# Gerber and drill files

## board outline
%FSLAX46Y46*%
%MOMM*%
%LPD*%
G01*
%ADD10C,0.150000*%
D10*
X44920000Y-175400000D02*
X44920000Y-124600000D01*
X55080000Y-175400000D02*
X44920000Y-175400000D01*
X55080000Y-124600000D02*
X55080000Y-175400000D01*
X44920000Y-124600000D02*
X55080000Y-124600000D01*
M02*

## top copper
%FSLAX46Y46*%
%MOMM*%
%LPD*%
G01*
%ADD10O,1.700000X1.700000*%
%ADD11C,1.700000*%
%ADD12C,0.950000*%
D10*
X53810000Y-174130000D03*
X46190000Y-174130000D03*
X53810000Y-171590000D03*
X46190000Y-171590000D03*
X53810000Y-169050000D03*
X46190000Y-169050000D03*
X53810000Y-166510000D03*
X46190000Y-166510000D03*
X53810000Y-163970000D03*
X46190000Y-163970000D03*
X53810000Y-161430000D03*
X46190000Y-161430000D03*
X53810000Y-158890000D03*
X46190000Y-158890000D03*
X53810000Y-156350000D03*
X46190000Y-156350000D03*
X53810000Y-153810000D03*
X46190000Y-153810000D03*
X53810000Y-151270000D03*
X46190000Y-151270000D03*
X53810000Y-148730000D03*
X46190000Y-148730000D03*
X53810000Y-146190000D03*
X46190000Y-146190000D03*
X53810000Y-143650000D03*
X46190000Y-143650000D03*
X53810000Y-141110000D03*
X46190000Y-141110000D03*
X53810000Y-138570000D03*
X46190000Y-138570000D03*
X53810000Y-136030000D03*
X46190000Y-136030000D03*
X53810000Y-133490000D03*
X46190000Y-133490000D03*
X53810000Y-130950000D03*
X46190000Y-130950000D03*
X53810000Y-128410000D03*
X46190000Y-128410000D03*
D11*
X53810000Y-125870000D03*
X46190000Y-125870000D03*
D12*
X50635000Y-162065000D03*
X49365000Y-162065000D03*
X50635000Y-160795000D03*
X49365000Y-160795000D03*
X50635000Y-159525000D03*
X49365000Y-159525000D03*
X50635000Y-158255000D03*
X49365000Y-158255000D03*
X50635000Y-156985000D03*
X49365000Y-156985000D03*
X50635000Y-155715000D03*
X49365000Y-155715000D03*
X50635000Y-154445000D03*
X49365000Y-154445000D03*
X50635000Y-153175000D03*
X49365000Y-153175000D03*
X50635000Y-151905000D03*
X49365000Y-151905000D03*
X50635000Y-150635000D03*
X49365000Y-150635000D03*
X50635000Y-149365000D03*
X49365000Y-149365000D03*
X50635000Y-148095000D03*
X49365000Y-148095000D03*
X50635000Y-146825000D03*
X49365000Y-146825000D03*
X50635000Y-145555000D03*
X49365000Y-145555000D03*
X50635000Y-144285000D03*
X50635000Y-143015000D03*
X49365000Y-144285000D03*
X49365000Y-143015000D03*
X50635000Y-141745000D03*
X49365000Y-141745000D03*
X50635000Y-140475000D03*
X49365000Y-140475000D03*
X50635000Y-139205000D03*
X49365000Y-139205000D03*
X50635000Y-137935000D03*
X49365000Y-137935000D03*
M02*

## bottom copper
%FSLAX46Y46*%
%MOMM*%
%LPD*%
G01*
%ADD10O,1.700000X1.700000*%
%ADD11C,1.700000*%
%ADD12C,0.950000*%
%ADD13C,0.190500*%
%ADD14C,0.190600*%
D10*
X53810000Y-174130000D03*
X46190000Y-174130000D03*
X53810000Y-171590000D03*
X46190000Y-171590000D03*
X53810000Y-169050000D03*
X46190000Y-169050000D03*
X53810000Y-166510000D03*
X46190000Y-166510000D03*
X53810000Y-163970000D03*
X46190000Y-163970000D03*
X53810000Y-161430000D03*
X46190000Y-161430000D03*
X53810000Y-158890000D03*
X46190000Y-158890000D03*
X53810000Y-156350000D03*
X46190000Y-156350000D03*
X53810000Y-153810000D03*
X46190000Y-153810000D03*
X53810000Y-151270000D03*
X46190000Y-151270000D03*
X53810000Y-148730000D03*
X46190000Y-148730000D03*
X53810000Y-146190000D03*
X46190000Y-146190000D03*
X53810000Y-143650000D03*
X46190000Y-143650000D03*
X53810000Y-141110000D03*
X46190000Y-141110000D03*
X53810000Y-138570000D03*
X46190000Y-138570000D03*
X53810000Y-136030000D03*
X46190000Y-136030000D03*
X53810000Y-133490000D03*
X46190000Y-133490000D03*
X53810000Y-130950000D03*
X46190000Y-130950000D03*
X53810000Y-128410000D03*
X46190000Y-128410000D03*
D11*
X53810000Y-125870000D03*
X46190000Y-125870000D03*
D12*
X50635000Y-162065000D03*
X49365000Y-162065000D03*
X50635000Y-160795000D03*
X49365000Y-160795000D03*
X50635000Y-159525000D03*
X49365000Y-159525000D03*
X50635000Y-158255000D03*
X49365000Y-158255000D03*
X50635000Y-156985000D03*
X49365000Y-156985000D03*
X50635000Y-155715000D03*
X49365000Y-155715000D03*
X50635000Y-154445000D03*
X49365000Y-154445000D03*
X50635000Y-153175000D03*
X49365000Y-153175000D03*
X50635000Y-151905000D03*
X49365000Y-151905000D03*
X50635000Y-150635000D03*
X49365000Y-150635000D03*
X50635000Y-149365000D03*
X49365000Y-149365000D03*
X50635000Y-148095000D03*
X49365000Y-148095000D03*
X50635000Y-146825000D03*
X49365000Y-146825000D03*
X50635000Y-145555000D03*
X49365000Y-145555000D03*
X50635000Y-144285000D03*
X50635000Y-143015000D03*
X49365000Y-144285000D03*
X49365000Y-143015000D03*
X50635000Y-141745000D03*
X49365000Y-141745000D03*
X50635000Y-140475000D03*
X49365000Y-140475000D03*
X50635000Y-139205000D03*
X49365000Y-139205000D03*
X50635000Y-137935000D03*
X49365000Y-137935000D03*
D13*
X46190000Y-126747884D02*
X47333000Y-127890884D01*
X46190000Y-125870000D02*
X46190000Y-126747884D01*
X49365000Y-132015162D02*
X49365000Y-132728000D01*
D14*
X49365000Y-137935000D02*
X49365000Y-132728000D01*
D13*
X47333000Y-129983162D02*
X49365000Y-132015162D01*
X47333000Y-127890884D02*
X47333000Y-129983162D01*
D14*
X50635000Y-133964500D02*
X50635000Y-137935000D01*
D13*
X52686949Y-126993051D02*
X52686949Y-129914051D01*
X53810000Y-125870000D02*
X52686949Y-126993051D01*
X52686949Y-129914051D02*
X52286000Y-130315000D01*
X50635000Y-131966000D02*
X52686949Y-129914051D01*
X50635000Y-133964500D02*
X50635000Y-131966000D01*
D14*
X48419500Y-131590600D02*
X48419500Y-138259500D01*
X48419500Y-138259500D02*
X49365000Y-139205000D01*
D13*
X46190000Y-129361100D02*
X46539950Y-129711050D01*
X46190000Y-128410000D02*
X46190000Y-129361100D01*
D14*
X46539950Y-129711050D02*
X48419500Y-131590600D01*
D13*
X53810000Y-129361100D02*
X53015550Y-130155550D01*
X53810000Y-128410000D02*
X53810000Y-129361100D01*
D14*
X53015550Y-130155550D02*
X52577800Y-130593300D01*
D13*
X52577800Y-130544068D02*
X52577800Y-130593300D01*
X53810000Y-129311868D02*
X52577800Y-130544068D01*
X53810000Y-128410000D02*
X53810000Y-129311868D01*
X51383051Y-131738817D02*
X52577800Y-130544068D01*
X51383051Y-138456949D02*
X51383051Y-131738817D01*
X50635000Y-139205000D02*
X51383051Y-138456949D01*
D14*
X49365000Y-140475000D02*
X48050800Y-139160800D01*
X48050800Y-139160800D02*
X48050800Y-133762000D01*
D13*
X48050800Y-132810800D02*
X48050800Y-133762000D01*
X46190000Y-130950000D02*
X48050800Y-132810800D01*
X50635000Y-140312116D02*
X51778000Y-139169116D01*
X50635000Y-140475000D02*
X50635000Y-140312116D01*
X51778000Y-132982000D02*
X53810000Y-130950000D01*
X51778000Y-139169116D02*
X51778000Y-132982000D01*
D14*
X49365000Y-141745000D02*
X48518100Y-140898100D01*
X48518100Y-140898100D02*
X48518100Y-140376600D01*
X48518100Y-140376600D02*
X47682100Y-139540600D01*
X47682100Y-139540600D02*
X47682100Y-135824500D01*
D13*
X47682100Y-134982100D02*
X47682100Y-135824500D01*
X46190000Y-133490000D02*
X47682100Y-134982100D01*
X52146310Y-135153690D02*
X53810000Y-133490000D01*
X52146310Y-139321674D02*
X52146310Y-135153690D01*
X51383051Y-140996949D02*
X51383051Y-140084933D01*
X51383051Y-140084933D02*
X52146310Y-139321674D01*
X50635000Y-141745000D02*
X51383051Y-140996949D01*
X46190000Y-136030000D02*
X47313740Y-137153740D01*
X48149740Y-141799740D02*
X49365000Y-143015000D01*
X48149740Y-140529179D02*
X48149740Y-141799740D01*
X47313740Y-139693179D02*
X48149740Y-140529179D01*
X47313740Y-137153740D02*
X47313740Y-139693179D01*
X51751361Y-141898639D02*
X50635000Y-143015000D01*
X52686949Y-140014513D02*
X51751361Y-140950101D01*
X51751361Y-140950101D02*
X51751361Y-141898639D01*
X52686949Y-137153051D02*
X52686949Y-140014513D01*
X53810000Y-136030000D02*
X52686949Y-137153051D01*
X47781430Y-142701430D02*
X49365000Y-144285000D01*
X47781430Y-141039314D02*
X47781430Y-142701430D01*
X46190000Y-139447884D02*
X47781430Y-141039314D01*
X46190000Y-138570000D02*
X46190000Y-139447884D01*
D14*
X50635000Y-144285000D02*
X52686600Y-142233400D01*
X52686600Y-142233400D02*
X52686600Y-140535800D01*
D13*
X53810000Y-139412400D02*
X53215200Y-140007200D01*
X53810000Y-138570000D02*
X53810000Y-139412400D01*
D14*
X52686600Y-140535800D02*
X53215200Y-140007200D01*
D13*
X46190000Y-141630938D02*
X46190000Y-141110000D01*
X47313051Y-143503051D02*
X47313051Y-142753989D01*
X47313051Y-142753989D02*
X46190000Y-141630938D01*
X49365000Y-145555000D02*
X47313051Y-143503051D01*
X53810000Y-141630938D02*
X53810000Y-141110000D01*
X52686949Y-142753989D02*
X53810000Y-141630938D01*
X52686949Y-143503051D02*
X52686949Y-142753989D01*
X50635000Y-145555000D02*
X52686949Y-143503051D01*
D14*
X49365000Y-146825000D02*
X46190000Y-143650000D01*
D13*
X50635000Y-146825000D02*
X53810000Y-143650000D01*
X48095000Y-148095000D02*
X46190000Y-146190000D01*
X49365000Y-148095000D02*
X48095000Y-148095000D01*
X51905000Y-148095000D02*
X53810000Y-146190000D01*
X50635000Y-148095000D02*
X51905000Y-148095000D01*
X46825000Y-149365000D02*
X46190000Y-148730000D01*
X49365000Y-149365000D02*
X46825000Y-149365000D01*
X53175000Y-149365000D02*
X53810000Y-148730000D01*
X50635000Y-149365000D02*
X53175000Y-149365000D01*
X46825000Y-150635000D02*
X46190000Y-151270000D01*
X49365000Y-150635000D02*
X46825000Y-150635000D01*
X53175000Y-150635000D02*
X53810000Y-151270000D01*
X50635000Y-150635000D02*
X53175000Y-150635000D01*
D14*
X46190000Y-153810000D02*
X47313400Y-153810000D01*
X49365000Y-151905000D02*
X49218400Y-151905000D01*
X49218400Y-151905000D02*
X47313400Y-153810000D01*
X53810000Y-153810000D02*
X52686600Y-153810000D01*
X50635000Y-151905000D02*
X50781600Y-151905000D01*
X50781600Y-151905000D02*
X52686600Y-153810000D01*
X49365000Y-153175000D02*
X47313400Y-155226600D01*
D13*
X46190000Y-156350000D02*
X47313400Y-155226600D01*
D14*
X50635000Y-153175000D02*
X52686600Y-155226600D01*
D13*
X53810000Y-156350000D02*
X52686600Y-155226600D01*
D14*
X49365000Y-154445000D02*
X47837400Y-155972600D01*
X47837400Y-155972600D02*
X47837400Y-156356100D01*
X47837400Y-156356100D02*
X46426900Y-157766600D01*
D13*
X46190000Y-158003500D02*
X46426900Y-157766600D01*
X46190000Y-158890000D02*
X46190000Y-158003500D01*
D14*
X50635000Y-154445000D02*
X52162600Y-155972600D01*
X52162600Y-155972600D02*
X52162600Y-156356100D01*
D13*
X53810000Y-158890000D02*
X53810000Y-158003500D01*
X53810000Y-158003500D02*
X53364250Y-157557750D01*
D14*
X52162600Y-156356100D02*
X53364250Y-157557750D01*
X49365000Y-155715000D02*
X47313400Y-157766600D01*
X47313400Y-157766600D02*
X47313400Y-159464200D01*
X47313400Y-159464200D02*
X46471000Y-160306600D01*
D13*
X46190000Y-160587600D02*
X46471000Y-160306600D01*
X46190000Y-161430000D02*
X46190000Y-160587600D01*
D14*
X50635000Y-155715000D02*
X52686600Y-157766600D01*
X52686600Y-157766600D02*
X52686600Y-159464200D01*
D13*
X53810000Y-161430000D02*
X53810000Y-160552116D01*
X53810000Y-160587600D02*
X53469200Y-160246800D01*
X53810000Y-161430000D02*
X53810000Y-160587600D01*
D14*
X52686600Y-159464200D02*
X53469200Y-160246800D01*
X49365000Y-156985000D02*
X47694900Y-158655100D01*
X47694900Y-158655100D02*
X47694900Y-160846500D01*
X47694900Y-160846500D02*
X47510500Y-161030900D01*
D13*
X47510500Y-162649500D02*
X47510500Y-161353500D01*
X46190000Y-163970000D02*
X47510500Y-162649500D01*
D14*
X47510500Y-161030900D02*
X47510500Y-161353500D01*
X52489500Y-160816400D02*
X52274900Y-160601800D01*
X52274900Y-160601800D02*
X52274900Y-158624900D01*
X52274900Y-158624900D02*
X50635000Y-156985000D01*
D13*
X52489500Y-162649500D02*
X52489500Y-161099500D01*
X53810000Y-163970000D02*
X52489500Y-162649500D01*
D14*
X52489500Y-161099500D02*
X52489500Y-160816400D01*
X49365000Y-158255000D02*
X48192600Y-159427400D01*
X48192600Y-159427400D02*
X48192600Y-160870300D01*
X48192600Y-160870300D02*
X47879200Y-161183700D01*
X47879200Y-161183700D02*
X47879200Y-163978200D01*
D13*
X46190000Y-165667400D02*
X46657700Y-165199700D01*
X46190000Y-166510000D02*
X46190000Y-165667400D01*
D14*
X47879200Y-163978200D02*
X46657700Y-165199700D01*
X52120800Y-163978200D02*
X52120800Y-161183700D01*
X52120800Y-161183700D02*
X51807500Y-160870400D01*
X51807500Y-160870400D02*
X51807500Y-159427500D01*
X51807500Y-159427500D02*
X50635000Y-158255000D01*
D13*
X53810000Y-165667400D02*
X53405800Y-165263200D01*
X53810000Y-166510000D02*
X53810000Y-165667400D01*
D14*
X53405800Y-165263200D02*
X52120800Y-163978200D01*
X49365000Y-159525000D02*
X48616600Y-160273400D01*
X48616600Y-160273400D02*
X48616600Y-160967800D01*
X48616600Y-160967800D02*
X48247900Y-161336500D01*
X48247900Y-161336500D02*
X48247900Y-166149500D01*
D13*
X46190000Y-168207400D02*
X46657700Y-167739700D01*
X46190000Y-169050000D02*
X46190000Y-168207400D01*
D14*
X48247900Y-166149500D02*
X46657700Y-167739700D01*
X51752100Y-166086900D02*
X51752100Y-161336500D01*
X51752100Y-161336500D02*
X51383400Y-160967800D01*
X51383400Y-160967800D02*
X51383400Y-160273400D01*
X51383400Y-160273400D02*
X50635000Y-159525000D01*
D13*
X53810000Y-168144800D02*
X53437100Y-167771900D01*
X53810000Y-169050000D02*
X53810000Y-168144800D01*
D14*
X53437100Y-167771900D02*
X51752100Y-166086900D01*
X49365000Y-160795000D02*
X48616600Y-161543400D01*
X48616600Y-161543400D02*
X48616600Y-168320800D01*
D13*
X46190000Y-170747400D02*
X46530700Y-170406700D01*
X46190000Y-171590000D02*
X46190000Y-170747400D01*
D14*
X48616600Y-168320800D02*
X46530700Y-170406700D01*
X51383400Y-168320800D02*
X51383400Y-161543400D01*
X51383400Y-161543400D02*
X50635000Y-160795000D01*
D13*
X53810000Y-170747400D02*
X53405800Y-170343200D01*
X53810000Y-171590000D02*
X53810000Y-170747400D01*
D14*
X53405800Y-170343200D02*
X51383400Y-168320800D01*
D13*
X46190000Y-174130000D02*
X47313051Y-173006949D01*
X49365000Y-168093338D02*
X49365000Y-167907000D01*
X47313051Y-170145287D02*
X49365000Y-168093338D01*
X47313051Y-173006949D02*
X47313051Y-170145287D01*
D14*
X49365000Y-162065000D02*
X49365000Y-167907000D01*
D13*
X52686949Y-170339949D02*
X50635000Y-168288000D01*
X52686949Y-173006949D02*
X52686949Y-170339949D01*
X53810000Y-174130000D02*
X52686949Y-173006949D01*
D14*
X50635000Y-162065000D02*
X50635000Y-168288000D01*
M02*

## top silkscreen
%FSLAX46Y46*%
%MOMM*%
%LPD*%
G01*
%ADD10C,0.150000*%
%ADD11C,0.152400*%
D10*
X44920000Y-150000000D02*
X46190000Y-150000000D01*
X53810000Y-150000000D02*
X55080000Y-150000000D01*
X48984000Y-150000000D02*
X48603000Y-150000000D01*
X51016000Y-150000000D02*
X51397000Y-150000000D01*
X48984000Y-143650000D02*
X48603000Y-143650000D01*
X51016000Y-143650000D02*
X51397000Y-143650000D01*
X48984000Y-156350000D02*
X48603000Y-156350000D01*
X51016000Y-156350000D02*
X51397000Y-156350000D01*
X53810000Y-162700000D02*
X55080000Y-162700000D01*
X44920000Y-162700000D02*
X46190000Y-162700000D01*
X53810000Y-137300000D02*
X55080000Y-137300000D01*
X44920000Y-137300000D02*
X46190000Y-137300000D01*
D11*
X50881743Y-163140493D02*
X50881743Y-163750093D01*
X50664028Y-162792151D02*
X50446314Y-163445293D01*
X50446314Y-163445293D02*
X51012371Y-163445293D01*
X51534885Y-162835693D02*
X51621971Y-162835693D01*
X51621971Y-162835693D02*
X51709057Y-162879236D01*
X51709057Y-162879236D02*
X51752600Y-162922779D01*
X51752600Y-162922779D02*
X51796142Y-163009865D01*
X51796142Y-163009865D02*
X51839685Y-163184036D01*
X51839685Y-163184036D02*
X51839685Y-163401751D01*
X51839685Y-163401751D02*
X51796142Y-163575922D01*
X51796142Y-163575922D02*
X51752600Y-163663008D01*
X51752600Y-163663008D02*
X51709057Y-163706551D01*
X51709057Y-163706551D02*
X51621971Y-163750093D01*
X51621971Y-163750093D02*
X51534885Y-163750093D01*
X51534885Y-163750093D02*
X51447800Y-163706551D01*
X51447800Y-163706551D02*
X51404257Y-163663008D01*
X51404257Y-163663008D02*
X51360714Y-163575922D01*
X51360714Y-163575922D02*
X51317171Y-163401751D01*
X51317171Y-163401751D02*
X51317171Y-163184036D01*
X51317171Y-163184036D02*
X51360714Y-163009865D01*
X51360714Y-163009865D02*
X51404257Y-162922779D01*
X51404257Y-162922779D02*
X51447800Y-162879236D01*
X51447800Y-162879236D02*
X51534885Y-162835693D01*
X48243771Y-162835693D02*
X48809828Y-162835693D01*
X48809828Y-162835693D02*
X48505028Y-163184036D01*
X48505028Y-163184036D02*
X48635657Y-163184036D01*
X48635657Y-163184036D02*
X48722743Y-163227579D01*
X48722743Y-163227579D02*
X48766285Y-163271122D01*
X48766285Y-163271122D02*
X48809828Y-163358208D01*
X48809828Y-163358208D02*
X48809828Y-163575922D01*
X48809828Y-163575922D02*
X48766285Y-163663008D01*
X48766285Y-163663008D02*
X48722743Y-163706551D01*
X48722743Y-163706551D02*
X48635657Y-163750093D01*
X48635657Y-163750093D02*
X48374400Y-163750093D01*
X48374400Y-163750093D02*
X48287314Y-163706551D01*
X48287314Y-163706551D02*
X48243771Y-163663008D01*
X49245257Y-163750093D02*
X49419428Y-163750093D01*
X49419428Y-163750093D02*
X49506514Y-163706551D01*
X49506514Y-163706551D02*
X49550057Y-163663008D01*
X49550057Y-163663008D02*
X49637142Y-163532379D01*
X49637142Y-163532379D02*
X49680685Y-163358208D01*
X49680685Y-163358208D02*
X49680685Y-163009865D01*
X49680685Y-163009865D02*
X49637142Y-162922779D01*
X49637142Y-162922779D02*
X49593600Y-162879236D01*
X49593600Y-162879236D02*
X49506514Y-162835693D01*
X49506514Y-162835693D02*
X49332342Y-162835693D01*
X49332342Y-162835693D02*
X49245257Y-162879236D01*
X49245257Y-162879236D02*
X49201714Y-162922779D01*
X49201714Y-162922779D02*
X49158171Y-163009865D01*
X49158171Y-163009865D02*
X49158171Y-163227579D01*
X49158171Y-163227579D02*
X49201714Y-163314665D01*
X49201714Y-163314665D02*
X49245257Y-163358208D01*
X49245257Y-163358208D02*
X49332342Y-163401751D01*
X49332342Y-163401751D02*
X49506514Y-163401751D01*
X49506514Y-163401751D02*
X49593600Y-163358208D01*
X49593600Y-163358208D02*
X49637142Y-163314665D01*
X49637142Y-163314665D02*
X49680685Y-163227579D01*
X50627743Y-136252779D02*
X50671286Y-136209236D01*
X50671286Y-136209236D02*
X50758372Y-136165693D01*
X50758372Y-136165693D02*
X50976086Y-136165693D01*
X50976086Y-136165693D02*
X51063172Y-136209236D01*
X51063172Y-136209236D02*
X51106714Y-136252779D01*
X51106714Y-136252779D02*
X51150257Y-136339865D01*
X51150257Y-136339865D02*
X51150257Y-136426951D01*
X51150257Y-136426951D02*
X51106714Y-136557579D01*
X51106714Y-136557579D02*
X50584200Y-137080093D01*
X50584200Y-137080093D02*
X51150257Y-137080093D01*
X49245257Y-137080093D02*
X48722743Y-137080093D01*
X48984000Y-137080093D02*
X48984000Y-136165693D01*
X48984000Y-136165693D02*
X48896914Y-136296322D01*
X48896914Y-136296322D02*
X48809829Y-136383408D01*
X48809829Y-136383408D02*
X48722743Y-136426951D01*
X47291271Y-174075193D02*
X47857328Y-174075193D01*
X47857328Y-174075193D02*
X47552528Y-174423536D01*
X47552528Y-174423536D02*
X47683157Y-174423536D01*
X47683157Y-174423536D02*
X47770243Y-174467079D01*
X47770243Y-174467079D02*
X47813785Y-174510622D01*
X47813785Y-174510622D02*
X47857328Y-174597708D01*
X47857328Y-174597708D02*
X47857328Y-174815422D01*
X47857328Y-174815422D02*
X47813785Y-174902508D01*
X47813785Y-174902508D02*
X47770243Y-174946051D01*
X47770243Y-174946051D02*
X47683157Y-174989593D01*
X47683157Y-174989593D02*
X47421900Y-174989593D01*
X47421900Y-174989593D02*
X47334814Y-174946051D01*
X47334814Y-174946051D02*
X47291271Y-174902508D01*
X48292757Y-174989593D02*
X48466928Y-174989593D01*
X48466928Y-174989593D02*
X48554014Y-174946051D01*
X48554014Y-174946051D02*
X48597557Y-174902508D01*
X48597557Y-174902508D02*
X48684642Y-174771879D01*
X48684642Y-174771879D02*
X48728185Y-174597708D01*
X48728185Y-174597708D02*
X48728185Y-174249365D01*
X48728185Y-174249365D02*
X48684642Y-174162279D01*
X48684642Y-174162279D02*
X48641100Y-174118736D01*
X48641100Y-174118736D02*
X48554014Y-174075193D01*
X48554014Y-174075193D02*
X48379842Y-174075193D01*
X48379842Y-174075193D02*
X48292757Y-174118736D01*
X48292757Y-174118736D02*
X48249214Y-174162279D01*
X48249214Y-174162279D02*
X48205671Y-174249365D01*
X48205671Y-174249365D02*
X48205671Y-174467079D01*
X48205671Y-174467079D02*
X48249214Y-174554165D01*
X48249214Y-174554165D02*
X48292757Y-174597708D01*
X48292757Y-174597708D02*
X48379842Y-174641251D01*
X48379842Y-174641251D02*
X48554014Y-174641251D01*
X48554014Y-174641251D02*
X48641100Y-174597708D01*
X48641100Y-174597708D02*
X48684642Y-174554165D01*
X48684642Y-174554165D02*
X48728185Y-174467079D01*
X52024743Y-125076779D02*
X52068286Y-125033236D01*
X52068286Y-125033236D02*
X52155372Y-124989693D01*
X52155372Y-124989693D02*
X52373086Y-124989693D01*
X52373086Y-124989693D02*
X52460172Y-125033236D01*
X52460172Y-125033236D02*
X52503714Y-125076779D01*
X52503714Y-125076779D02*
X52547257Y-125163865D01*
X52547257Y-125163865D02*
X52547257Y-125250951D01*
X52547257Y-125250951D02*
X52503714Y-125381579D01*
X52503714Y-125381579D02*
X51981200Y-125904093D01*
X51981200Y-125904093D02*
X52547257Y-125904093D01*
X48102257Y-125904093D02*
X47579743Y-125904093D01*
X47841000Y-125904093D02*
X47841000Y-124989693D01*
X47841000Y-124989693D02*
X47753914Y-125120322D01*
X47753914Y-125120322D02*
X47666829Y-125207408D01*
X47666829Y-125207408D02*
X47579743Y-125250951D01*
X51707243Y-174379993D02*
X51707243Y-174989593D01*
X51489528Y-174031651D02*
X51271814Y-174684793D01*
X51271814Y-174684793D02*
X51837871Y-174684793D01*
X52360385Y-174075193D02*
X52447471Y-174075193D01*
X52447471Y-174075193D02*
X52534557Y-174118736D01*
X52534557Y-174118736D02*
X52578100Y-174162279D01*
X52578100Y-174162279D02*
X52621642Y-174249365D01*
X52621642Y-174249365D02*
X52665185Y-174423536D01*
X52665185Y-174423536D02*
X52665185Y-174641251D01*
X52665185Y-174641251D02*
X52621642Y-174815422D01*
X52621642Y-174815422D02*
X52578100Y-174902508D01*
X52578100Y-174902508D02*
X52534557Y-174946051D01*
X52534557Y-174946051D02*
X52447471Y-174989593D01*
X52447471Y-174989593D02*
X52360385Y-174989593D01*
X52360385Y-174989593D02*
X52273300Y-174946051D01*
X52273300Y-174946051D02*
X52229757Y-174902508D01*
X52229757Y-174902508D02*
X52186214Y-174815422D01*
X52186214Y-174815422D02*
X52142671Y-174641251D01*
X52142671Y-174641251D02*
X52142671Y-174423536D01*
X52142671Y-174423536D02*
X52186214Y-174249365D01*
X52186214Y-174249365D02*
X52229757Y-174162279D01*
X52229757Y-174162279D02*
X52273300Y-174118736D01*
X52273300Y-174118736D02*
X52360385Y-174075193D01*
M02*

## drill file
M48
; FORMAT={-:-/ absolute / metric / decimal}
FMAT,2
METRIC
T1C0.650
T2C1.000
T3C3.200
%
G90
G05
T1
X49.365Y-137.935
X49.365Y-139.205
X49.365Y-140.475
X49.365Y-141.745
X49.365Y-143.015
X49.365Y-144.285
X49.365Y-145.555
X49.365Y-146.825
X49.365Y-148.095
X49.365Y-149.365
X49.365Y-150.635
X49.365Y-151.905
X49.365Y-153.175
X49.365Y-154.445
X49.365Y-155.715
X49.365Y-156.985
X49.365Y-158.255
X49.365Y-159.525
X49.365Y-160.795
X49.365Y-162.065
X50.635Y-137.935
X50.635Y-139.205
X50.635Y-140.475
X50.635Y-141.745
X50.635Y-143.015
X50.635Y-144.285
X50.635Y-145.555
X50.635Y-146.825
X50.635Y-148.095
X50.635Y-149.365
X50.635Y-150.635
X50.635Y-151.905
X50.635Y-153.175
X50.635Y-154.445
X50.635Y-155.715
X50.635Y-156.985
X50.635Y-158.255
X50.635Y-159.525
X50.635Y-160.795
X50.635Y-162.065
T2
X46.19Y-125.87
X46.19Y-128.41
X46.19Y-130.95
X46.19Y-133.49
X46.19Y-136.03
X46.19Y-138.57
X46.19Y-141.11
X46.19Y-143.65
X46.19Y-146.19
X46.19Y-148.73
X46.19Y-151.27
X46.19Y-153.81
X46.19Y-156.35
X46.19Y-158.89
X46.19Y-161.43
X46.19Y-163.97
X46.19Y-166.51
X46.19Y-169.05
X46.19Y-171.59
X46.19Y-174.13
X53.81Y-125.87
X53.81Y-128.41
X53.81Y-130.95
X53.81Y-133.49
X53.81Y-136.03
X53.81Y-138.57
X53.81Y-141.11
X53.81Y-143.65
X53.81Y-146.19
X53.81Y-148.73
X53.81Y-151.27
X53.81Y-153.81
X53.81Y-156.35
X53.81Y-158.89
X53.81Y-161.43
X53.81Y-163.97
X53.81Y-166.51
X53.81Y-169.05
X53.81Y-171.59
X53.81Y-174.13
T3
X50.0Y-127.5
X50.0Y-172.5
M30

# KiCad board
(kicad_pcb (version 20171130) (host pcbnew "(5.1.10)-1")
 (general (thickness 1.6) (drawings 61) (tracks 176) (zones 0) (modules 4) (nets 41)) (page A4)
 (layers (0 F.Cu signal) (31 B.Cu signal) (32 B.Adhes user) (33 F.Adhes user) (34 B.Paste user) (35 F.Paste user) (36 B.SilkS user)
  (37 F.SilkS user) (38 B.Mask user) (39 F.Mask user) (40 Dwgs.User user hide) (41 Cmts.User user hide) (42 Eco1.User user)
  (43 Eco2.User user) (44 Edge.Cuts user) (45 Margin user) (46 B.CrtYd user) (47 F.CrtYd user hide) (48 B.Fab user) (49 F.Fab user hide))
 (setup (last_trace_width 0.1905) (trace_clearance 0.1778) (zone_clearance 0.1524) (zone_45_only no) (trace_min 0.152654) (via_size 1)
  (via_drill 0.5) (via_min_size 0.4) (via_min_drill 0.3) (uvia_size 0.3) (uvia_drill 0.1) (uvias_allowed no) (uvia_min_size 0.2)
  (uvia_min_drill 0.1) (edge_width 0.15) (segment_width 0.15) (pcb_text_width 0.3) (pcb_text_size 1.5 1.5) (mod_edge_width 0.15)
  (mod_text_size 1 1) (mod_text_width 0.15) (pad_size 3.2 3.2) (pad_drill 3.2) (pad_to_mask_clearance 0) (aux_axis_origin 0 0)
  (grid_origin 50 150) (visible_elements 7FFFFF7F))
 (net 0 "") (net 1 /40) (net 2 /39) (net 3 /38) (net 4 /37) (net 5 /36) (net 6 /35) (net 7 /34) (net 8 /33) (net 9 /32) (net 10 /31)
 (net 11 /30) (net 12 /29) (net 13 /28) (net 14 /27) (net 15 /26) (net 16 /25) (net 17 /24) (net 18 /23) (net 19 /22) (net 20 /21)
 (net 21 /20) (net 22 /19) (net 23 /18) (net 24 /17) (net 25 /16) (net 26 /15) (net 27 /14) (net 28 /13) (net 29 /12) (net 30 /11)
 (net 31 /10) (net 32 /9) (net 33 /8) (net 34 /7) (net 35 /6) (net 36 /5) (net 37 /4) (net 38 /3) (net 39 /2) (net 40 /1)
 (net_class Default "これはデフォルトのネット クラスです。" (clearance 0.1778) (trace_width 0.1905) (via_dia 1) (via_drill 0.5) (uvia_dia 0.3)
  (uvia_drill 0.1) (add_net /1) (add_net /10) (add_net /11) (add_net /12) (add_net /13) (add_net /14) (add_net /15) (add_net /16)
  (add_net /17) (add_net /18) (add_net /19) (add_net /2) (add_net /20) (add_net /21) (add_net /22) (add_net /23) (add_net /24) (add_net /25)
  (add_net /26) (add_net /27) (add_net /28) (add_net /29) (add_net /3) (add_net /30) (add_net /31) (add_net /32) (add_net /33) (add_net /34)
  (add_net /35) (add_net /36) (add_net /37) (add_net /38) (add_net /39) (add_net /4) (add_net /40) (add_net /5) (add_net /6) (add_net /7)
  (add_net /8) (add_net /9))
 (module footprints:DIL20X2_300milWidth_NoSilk (layer F.Cu) (at 50 150)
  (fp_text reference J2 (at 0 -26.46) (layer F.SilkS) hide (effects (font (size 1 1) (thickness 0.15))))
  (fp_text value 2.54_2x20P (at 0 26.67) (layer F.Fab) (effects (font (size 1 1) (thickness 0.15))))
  (pad 40 thru_hole oval (at 3.81 24.13) (size 1.7 1.7) (drill 1) (layers *.Cu *.Mask) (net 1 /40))
  (pad 39 thru_hole oval (at -3.81 24.13) (size 1.7 1.7) (drill 1) (layers *.Cu *.Mask) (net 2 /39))
  (pad 38 thru_hole oval (at 3.81 21.59) (size 1.7 1.7) (drill 1) (layers *.Cu *.Mask) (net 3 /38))
  (pad 37 thru_hole oval (at -3.81 21.59) (size 1.7 1.7) (drill 1) (layers *.Cu *.Mask) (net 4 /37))
  (pad 36 thru_hole oval (at 3.81 19.05) (size 1.7 1.7) (drill 1) (layers *.Cu *.Mask) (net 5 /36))
  (pad 35 thru_hole oval (at -3.81 19.05) (size 1.7 1.7) (drill 1) (layers *.Cu *.Mask) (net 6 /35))
  (pad 34 thru_hole oval (at 3.81 16.51) (size 1.7 1.7) (drill 1) (layers *.Cu *.Mask) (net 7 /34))
  (pad 33 thru_hole oval (at -3.81 16.51) (size 1.7 1.7) (drill 1) (layers *.Cu *.Mask) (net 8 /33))
  (pad 32 thru_hole oval (at 3.81 13.97) (size 1.7 1.7) (drill 1) (layers *.Cu *.Mask) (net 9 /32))
  (pad 31 thru_hole oval (at -3.81 13.97) (size 1.7 1.7) (drill 1) (layers *.Cu *.Mask) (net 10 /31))
  (pad 30 thru_hole oval (at 3.81 11.43) (size 1.7 1.7) (drill 1) (layers *.Cu *.Mask) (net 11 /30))
  (pad 29 thru_hole oval (at -3.81 11.43) (size 1.7 1.7) (drill 1) (layers *.Cu *.Mask) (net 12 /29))
  (pad 28 thru_hole oval (at 3.81 8.89) (size 1.7 1.7) (drill 1) (layers *.Cu *.Mask) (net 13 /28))
  (pad 27 thru_hole oval (at -3.81 8.89) (size 1.7 1.7) (drill 1) (layers *.Cu *.Mask) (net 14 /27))
  (pad 26 thru_hole oval (at 3.81 6.35) (size 1.7 1.7) (drill 1) (layers *.Cu *.Mask) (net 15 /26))
  (pad 25 thru_hole oval (at -3.81 6.35) (size 1.7 1.7) (drill 1) (layers *.Cu *.Mask) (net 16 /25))
  (pad 24 thru_hole oval (at 3.81 3.81) (size 1.7 1.7) (drill 1) (layers *.Cu *.Mask) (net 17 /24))
  (pad 23 thru_hole oval (at -3.81 3.81) (size 1.7 1.7) (drill 1) (layers *.Cu *.Mask) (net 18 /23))
  (pad 22 thru_hole oval (at 3.81 1.27) (size 1.7 1.7) (drill 1) (layers *.Cu *.Mask) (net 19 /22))
  (pad 21 thru_hole oval (at -3.81 1.27) (size 1.7 1.7) (drill 1) (layers *.Cu *.Mask) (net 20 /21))
  (pad 20 thru_hole oval (at 3.81 -1.27) (size 1.7 1.7) (drill 1) (layers *.Cu *.Mask) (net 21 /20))
  (pad 19 thru_hole oval (at -3.81 -1.27) (size 1.7 1.7) (drill 1) (layers *.Cu *.Mask) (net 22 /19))
  (pad 18 thru_hole oval (at 3.81 -3.81) (size 1.7 1.7) (drill 1) (layers *.Cu *.Mask) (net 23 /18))
  (pad 17 thru_hole oval (at -3.81 -3.81) (size 1.7 1.7) (drill 1) (layers *.Cu *.Mask) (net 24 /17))
  (pad 16 thru_hole oval (at 3.81 -6.35) (size 1.7 1.7) (drill 1) (layers *.Cu *.Mask) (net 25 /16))
  (pad 15 thru_hole oval (at -3.81 -6.35) (size 1.7 1.7) (drill 1) (layers *.Cu *.Mask) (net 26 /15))
  (pad 14 thru_hole oval (at 3.81 -8.89) (size 1.7 1.7) (drill 1) (layers *.Cu *.Mask) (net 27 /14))
  (pad 13 thru_hole oval (at -3.81 -8.89) (size 1.7 1.7) (drill 1) (layers *.Cu *.Mask) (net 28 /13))
  (pad 12 thru_hole oval (at 3.81 -11.43) (size 1.7 1.7) (drill 1) (layers *.Cu *.Mask) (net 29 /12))
  (pad 11 thru_hole oval (at -3.81 -11.43) (size 1.7 1.7) (drill 1) (layers *.Cu *.Mask) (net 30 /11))
  (pad 10 thru_hole oval (at 3.81 -13.97) (size 1.7 1.7) (drill 1) (layers *.Cu *.Mask) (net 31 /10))
  (pad 9 thru_hole oval (at -3.81 -13.97) (size 1.7 1.7) (drill 1) (layers *.Cu *.Mask) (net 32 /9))
  (pad 8 thru_hole oval (at 3.81 -16.51) (size 1.7 1.7) (drill 1) (layers *.Cu *.Mask) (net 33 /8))
  (pad 7 thru_hole oval (at -3.81 -16.51) (size 1.7 1.7) (drill 1) (layers *.Cu *.Mask) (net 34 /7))
  (pad 6 thru_hole oval (at 3.81 -19.05) (size 1.7 1.7) (drill 1) (layers *.Cu *.Mask) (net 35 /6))
  (pad 5 thru_hole oval (at -3.81 -19.05) (size 1.7 1.7) (drill 1) (layers *.Cu *.Mask) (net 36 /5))
  (pad 4 thru_hole oval (at 3.81 -21.59) (size 1.7 1.7) (drill 1) (layers *.Cu *.Mask) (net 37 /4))
  (pad 3 thru_hole oval (at -3.81 -21.59) (size 1.7 1.7) (drill 1) (layers *.Cu *.Mask) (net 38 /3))
  (pad 2 thru_hole circle (at 3.81 -24.13) (size 1.7 1.7) (drill 1) (layers *.Cu *.Mask) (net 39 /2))
  (pad 1 thru_hole circle (at -3.81 -24.13) (size 1.7 1.7) (drill 1) (layers *.Cu *.Mask) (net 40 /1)))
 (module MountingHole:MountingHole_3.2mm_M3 (layer F.Cu) (at 50 127)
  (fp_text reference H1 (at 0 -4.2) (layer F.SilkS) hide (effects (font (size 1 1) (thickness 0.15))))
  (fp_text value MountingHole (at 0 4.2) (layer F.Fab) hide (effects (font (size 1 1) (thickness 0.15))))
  (pad "" np_thru_hole circle (at 0 0.5) (size 3.2 3.2) (drill 3.2) (layers *.Cu *.Mask)))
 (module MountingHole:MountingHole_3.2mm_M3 (layer F.Cu) (at 50 173)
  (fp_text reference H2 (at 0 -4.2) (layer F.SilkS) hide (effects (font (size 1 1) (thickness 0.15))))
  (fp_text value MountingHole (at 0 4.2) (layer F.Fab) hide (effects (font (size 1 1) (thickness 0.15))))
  (pad "" np_thru_hole circle (at 0 -0.5) (size 3.2 3.2) (drill 3.2) (layers *.Cu *.Mask)))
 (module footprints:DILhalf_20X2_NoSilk (layer F.Cu) (at 50 150)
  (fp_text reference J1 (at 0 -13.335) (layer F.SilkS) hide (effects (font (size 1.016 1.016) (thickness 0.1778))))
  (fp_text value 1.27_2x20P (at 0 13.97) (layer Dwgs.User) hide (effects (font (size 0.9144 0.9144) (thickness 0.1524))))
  (pad 40 thru_hole circle (at 0.635 12.065) (size 0.95 0.95) (drill 0.65) (layers *.Cu *.Mask) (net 1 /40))
  (pad 39 thru_hole circle (at -0.635 12.065) (size 0.95 0.95) (drill 0.65) (layers *.Cu *.Mask) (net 2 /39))
  (pad 38 thru_hole circle (at 0.635 10.795) (size 0.95 0.95) (drill 0.65) (layers *.Cu *.Mask) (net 3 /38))
  (pad 37 thru_hole circle (at -0.635 10.795) (size 0.95 0.95) (drill 0.65) (layers *.Cu *.Mask) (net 4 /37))
  (pad 36 thru_hole circle (at 0.635 9.525) (size 0.95 0.95) (drill 0.65) (layers *.Cu *.Mask) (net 5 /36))
  (pad 35 thru_hole circle (at -0.635 9.525) (size 0.95 0.95) (drill 0.65) (layers *.Cu *.Mask) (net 6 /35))
  (pad 34 thru_hole circle (at 0.635 8.255) (size 0.95 0.95) (drill 0.65) (layers *.Cu *.Mask) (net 7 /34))
  (pad 33 thru_hole circle (at -0.635 8.255) (size 0.95 0.95) (drill 0.65) (layers *.Cu *.Mask) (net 8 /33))
  (pad 32 thru_hole circle (at 0.635 6.985) (size 0.95 0.95) (drill 0.65) (layers *.Cu *.Mask) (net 9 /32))
  (pad 31 thru_hole circle (at -0.635 6.985) (size 0.95 0.95) (drill 0.65) (layers *.Cu *.Mask) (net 10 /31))
  (pad 30 thru_hole circle (at 0.635 5.715) (size 0.95 0.95) (drill 0.65) (layers *.Cu *.Mask) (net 11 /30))
  (pad 29 thru_hole circle (at -0.635 5.715) (size 0.95 0.95) (drill 0.65) (layers *.Cu *.Mask) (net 12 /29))
  (pad 28 thru_hole circle (at 0.635 4.445) (size 0.95 0.95) (drill 0.65) (layers *.Cu *.Mask) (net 13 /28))
  (pad 27 thru_hole circle (at -0.635 4.445) (size 0.95 0.95) (drill 0.65) (layers *.Cu *.Mask) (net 14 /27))
  (pad 26 thru_hole circle (at 0.635 3.175) (size 0.95 0.95) (drill 0.65) (layers *.Cu *.Mask) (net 15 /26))
  (pad 25 thru_hole circle (at -0.635 3.175) (size 0.95 0.95) (drill 0.65) (layers *.Cu *.Mask) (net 16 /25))
  (pad 24 thru_hole circle (at 0.635 1.905) (size 0.95 0.95) (drill 0.65) (layers *.Cu *.Mask) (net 17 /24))
  (pad 23 thru_hole circle (at -0.635 1.905) (size 0.95 0.95) (drill 0.65) (layers *.Cu *.Mask) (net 18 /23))
  (pad 22 thru_hole circle (at 0.635 0.635) (size 0.95 0.95) (drill 0.65) (layers *.Cu *.Mask) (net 19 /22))
  (pad 21 thru_hole circle (at -0.635 0.635) (size 0.95 0.95) (drill 0.65) (layers *.Cu *.Mask) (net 20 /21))
  (pad 20 thru_hole circle (at 0.635 -0.635) (size 0.95 0.95) (drill 0.65) (layers *.Cu *.Mask) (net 21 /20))
  (pad 19 thru_hole circle (at -0.635 -0.635) (size 0.95 0.95) (drill 0.65) (layers *.Cu *.Mask) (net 22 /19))
  (pad 18 thru_hole circle (at 0.635 -1.905) (size 0.95 0.95) (drill 0.65) (layers *.Cu *.Mask) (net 23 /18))
  (pad 17 thru_hole circle (at -0.635 -1.905) (size 0.95 0.95) (drill 0.65) (layers *.Cu *.Mask) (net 24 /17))
  (pad 16 thru_hole circle (at 0.635 -3.175) (size 0.95 0.95) (drill 0.65) (layers *.Cu *.Mask) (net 25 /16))
  (pad 15 thru_hole circle (at -0.635 -3.175) (size 0.95 0.95) (drill 0.65) (layers *.Cu *.Mask) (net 26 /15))
  (pad 14 thru_hole circle (at 0.635 -4.445) (size 0.95 0.95) (drill 0.65) (layers *.Cu *.Mask) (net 27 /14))
  (pad 13 thru_hole circle (at -0.635 -4.445) (size 0.95 0.95) (drill 0.65) (layers *.Cu *.Mask) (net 28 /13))
  (pad 12 thru_hole circle (at 0.635 -5.715) (size 0.95 0.95) (drill 0.65) (layers *.Cu *.Mask) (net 29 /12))
  (pad 10 thru_hole circle (at 0.635 -6.985) (size 0.95 0.95) (drill 0.65) (layers *.Cu *.Mask) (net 31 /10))
  (pad 11 thru_hole circle (at -0.635 -5.715) (size 0.95 0.95) (drill 0.65) (layers *.Cu *.Mask) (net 30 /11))
  (pad 9 thru_hole circle (at -0.635 -6.985) (size 0.95 0.95) (drill 0.65) (layers *.Cu *.Mask) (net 32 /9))
  (pad 8 thru_hole circle (at 0.635 -8.255) (size 0.95 0.95) (drill 0.65) (layers *.Cu *.Mask) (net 33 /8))
  (pad 7 thru_hole circle (at -0.635 -8.255) (size 0.95 0.95) (drill 0.65) (layers *.Cu *.Mask) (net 34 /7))
  (pad 6 thru_hole circle (at 0.635 -9.525) (size 0.95 0.95) (drill 0.65) (layers *.Cu *.Mask) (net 35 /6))
  (pad 5 thru_hole circle (at -0.635 -9.525) (size 0.95 0.95) (drill 0.65) (layers *.Cu *.Mask) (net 36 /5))
  (pad 4 thru_hole circle (at 0.635 -10.795) (size 0.95 0.95) (drill 0.65) (layers *.Cu *.Mask) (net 37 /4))
  (pad 3 thru_hole circle (at -0.635 -10.795) (size 0.95 0.95) (drill 0.65) (layers *.Cu *.Mask) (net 38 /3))
  (pad 2 thru_hole circle (at 0.635 -12.065) (size 0.95 0.95) (drill 0.65) (layers *.Cu *.Mask) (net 39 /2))
  (pad 1 thru_hole circle (at -0.635 -12.065) (size 0.95 0.95) (drill 0.65) (layers *.Cu *.Mask) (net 40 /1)))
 (gr_line (start 44.92 150) (end 46.19 150) (layer F.SilkS) (width 0.15))
 (gr_line (start 53.81 150) (end 55.08 150) (layer F.SilkS) (width 0.15))
 (gr_line (start 48.984 150) (end 48.603 150) (layer F.SilkS) (width 0.15))
 (gr_line (start 51.016 150) (end 51.397 150) (layer F.SilkS) (width 0.15))
 (gr_line (start 48.984 143.65) (end 48.603 143.65) (layer F.SilkS) (width 0.15))
 (gr_line (start 51.016 143.65) (end 51.397 143.65) (layer F.SilkS) (width 0.15))
 (gr_line (start 48.984 156.35) (end 48.603 156.35) (layer F.SilkS) (width 0.15))
 (gr_line (start 51.016 156.35) (end 51.397 156.35) (layer F.SilkS) (width 0.15))
 (gr_line (start 53.81 162.7) (end 55.08 162.7) (layer F.SilkS) (width 0.15))
 (gr_line (start 44.92 162.7) (end 46.19 162.7) (layer F.SilkS) (width 0.15))
 (gr_line (start 53.81 137.3) (end 55.08 137.3) (layer F.SilkS) (width 0.15))
 (gr_line (start 44.92 137.3) (end 46.19 137.3) (layer F.SilkS) (width 0.15))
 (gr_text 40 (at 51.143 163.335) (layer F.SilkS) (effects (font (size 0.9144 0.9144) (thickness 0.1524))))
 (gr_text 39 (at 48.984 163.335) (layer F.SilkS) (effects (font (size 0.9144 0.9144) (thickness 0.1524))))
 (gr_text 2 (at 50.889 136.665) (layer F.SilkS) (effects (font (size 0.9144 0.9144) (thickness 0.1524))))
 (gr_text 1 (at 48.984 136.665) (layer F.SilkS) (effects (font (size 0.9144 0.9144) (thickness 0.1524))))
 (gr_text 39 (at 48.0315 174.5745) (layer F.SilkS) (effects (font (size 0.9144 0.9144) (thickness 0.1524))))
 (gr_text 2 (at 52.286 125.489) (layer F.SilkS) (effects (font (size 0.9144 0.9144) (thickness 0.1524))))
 (gr_line (start 44.92 175.4) (end 44.92 124.6) (layer Edge.Cuts) (width 0.15))
 (gr_line (start 55.08 175.4) (end 44.92 175.4) (layer Edge.Cuts) (width 0.15))
 (gr_line (start 55.08 124.6) (end 55.08 175.4) (layer Edge.Cuts) (width 0.15))
 (gr_line (start 44.92 124.6) (end 55.08 124.6) (layer Edge.Cuts) (width 0.15))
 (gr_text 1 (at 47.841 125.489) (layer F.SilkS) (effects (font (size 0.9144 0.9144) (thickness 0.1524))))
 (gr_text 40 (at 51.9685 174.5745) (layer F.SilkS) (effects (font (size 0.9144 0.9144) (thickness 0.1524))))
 (segment (start 46.19 126.747884) (end 47.333 127.890884) (width 0.1905) (layer B.Cu) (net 40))
 (segment (start 46.19 125.87) (end 46.19 126.747884) (width 0.1905) (layer B.Cu) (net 40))
 (segment (start 49.365 132.015162) (end 49.365 132.728) (width 0.1905) (layer B.Cu) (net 40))
 (segment (start 49.365 137.935) (end 49.365 132.728) (width 0.1906) (layer B.Cu) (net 40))
 (segment (start 47.333 129.983162) (end 49.365 132.015162) (width 0.1905) (layer B.Cu) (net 40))
 (segment (start 47.333 127.890884) (end 47.333 129.983162) (width 0.1905) (layer B.Cu) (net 40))
 (segment (start 50.635 133.9645) (end 50.635 137.935) (width 0.1906) (layer B.Cu) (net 39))
 (segment (start 52.686949 126.993051) (end 52.686949 129.914051) (width 0.1905) (layer B.Cu) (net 39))
 (segment (start 53.81 125.87) (end 52.686949 126.993051) (width 0.1905) (layer B.Cu) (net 39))
 (segment (start 52.686949 129.914051) (end 52.286 130.315) (width 0.1905) (layer B.Cu) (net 39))
 (segment (start 50.635 131.966) (end 52.686949 129.914051) (width 0.1905) (layer B.Cu) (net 39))
 (segment (start 50.635 133.9645) (end 50.635 131.966) (width 0.1905) (layer B.Cu) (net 39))
 (segment (start 48.4195 131.5906) (end 48.4195 138.2595) (width 0.1906) (layer B.Cu) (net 38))
 (segment (start 48.4195 138.2595) (end 49.365 139.205) (width 0.1906) (layer B.Cu) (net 38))
 (segment (start 46.19 129.3611) (end 46.53995 129.71105) (width 0.1905) (layer B.Cu) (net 38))
 (segment (start 46.19 128.41) (end 46.19 129.3611) (width 0.1905) (layer B.Cu) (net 38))
 (segment (start 46.53995 129.71105) (end 48.4195 131.5906) (width 0.1906) (layer B.Cu) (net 38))
 (segment (start 53.81 129.3611) (end 53.01555 130.15555) (width 0.1905) (layer B.Cu) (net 37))
 (segment (start 53.81 128.41) (end 53.81 129.3611) (width 0.1905) (layer B.Cu) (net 37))
 (segment (start 53.01555 130.15555) (end 52.5778 130.5933) (width 0.1906) (layer B.Cu) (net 37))
 (segment (start 52.5778 130.544068) (end 52.5778 130.5933) (width 0.1905) (layer B.Cu) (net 37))
 (segment (start 53.81 129.311868) (end 52.5778 130.544068) (width 0.1905) (layer B.Cu) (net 37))
 (segment (start 53.81 128.41) (end 53.81 129.311868) (width 0.1905) (layer B.Cu) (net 37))
 (segment (start 51.383051 131.738817) (end 52.5778 130.544068) (width 0.1905) (layer B.Cu) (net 37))
 (segment (start 51.383051 138.456949) (end 51.383051 131.738817) (width 0.1905) (layer B.Cu) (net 37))
 (segment (start 50.635 139.205) (end 51.383051 138.456949) (width 0.1905) (layer B.Cu) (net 37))
 (segment (start 49.365 140.475) (end 48.0508 139.1608) (width 0.1906) (layer B.Cu) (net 36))
 (segment (start 48.0508 139.1608) (end 48.0508 133.762) (width 0.1906) (layer B.Cu) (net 36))
 (segment (start 48.0508 132.8108) (end 48.0508 133.762) (width 0.1905) (layer B.Cu) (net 36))
 (segment (start 46.19 130.95) (end 48.0508 132.8108) (width 0.1905) (layer B.Cu) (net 36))
 (segment (start 50.635 140.312116) (end 51.778 139.169116) (width 0.1905) (layer B.Cu) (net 35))
 (segment (start 50.635 140.475) (end 50.635 140.312116) (width 0.1905) (layer B.Cu) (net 35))
 (segment (start 51.778 132.982) (end 53.81 130.95) (width 0.1905) (layer B.Cu) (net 35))
 (segment (start 51.778 139.169116) (end 51.778 132.982) (width 0.1905) (layer B.Cu) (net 35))
 (segment (start 49.365 141.745) (end 48.5181 140.8981) (width 0.1906) (layer B.Cu) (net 34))
 (segment (start 48.5181 140.8981) (end 48.5181 140.3766) (width 0.1906) (layer B.Cu) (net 34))
 (segment (start 48.5181 140.3766) (end 47.6821 139.5406) (width 0.1906) (layer B.Cu) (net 34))
 (segment (start 47.6821 139.5406) (end 47.6821 135.8245) (width 0.1906) (layer B.Cu) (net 34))
 (segment (start 47.6821 134.9821) (end 47.6821 135.8245) (width 0.1905) (layer B.Cu) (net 34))
 (segment (start 46.19 133.49) (end 47.6821 134.9821) (width 0.1905) (layer B.Cu) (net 34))
 (segment (start 52.14631 135.15369) (end 53.81 133.49) (width 0.1905) (layer B.Cu) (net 33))
 (segment (start 52.14631 139.321674) (end 52.14631 135.15369) (width 0.1905) (layer B.Cu) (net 33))
 (segment (start 51.383051 140.996949) (end 51.383051 140.084933) (width 0.1905) (layer B.Cu) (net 33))
 (segment (start 51.383051 140.084933) (end 52.14631 139.321674) (width 0.1905) (layer B.Cu) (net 33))
 (segment (start 50.635 141.745) (end 51.383051 140.996949) (width 0.1905) (layer B.Cu) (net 33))
 (segment (start 46.19 136.03) (end 47.31374 137.15374) (width 0.1905) (layer B.Cu) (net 32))
 (segment (start 48.14974 141.79974) (end 49.365 143.015) (width 0.1905) (layer B.Cu) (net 32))
 (segment (start 48.14974 140.529179) (end 48.14974 141.79974) (width 0.1905) (layer B.Cu) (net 32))
 (segment (start 47.31374 139.693179) (end 48.14974 140.529179) (width 0.1905) (layer B.Cu) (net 32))
 (segment (start 47.31374 137.15374) (end 47.31374 139.693179) (width 0.1905) (layer B.Cu) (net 32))
 (segment (start 51.751361 141.898639) (end 50.635 143.015) (width 0.1905) (layer B.Cu) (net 31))
 (segment (start 52.686949 140.014513) (end 51.751361 140.950101) (width 0.1905) (layer B.Cu) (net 31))
 (segment (start 51.751361 140.950101) (end 51.751361 141.898639) (width 0.1905) (layer B.Cu) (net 31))
 (segment (start 52.686949 137.153051) (end 52.686949 140.014513) (width 0.1905) (layer B.Cu) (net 31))
 (segment (start 53.81 136.03) (end 52.686949 137.153051) (width 0.1905) (layer B.Cu) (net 31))
 (segment (start 47.78143 142.70143) (end 49.365 144.285) (width 0.1905) (layer B.Cu) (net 30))
 (segment (start 47.78143 141.039314) (end 47.78143 142.70143) (width 0.1905) (layer B.Cu) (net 30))
 (segment (start 46.19 139.447884) (end 47.78143 141.039314) (width 0.1905) (layer B.Cu) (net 30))
 (segment (start 46.19 138.57) (end 46.19 139.447884) (width 0.1905) (layer B.Cu) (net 30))
 (segment (start 50.635 144.285) (end 52.6866 142.2334) (width 0.1906) (layer B.Cu) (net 29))
 (segment (start 52.6866 142.2334) (end 52.6866 140.5358) (width 0.1906) (layer B.Cu) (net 29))
 (segment (start 53.81 139.4124) (end 53.2152 140.0072) (width 0.1905) (layer B.Cu) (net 29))
 (segment (start 53.81 138.57) (end 53.81 139.4124) (width 0.1905) (layer B.Cu) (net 29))
 (segment (start 52.6866 140.5358) (end 53.2152 140.0072) (width 0.1906) (layer B.Cu) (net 29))
 (segment (start 46.19 141.630938) (end 46.19 141.11) (width 0.1905) (layer B.Cu) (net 28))
 (segment (start 47.313051 143.503051) (end 47.313051 142.753989) (width 0.1905) (layer B.Cu) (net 28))
 (segment (start 47.313051 142.753989) (end 46.19 141.630938) (width 0.1905) (layer B.Cu) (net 28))
 (segment (start 49.365 145.555) (end 47.313051 143.503051) (width 0.1905) (layer B.Cu) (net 28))
 (segment (start 53.81 141.630938) (end 53.81 141.11) (width 0.1905) (layer B.Cu) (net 27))
 (segment (start 52.686949 142.753989) (end 53.81 141.630938) (width 0.1905) (layer B.Cu) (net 27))
 (segment (start 52.686949 143.503051) (end 52.686949 142.753989) (width 0.1905) (layer B.Cu) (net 27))
 (segment (start 50.635 145.555) (end 52.686949 143.503051) (width 0.1905) (layer B.Cu) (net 27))
 (segment (start 49.365 146.825) (end 46.19 143.65) (width 0.1906) (layer B.Cu) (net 26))
 (segment (start 50.635 146.825) (end 53.81 143.65) (width 0.1905) (layer B.Cu) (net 25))
 (segment (start 48.095 148.095) (end 46.19 146.19) (width 0.1905) (layer B.Cu) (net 24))
 (segment (start 49.365 148.095) (end 48.095 148.095) (width 0.1905) (layer B.Cu) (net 24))
 (segment (start 51.905 148.095) (end 53.81 146.19) (width 0.1905) (layer B.Cu) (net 23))
 (segment (start 50.635 148.095) (end 51.905 148.095) (width 0.1905) (layer B.Cu) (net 23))
 (segment (start 46.825 149.365) (end 46.19 148.73) (width 0.1905) (layer B.Cu) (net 22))
 (segment (start 49.365 149.365) (end 46.825 149.365) (width 0.1905) (layer B.Cu) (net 22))
 (segment (start 53.175 149.365) (end 53.81 148.73) (width 0.1905) (layer B.Cu) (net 21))
 (segment (start 50.635 149.365) (end 53.175 149.365) (width 0.1905) (layer B.Cu) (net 21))
 (segment (start 46.825 150.635) (end 46.19 151.27) (width 0.1905) (layer B.Cu) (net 20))
 (segment (start 49.365 150.635) (end 46.825 150.635) (width 0.1905) (layer B.Cu) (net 20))
 (segment (start 53.175 150.635) (end 53.81 151.27) (width 0.1905) (layer B.Cu) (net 19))
 (segment (start 50.635 150.635) (end 53.175 150.635) (width 0.1905) (layer B.Cu) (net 19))
 (segment (start 46.19 153.81) (end 47.3134 153.81) (width 0.1906) (layer B.Cu) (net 18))
 (segment (start 49.365 151.905) (end 49.2184 151.905) (width 0.1906) (layer B.Cu) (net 18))
 (segment (start 49.2184 151.905) (end 47.3134 153.81) (width 0.1906) (layer B.Cu) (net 18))
 (segment (start 53.81 153.81) (end 52.6866 153.81) (width 0.1906) (layer B.Cu) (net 17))
 (segment (start 50.635 151.905) (end 50.7816 151.905) (width 0.1906) (layer B.Cu) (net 17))
 (segment (start 50.7816 151.905) (end 52.6866 153.81) (width 0.1906) (layer B.Cu) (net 17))
 (segment (start 49.365 153.175) (end 47.3134 155.2266) (width 0.1906) (layer B.Cu) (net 16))
 (segment (start 46.19 156.35) (end 47.3134 155.2266) (width 0.1905) (layer B.Cu) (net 16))
 (segment (start 50.635 153.175) (end 52.6866 155.2266) (width 0.1906) (layer B.Cu) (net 15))
 (segment (start 53.81 156.35) (end 52.6866 155.2266) (width 0.1905) (layer B.Cu) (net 15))
 (segment (start 49.365 154.445) (end 47.8374 155.9726) (width 0.1906) (layer B.Cu) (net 14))
 (segment (start 47.8374 155.9726) (end 47.8374 156.3561) (width 0.1906) (layer B.Cu) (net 14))
 (segment (start 47.8374 156.3561) (end 46.4269 157.7666) (width 0.1906) (layer B.Cu) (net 14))
 (segment (start 46.19 158.0035) (end 46.4269 157.7666) (width 0.1905) (layer B.Cu) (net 14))
 (segment (start 46.19 158.89) (end 46.19 158.0035) (width 0.1905) (layer B.Cu) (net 14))
 (segment (start 50.635 154.445) (end 52.1626 155.9726) (width 0.1906) (layer B.Cu) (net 13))
 (segment (start 52.1626 155.9726) (end 52.1626 156.3561) (width 0.1906) (layer B.Cu) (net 13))
 (segment (start 53.81 158.89) (end 53.81 158.0035) (width 0.1905) (layer B.Cu) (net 13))
 (segment (start 53.81 158.0035) (end 53.36425 157.55775) (width 0.1905) (layer B.Cu) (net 13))
 (segment (start 52.1626 156.3561) (end 53.36425 157.55775) (width 0.1906) (layer B.Cu) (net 13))
 (segment (start 49.365 155.715) (end 47.3134 157.7666) (width 0.1906) (layer B.Cu) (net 12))
 (segment (start 47.3134 157.7666) (end 47.3134 159.4642) (width 0.1906) (layer B.Cu) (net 12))
 (segment (start 47.3134 159.4642) (end 46.471 160.3066) (width 0.1906) (layer B.Cu) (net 12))
 (segment (start 46.19 160.5876) (end 46.471 160.3066) (width 0.1905) (layer B.Cu) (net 12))
 (segment (start 46.19 161.43) (end 46.19 160.5876) (width 0.1905) (layer B.Cu) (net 12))
 (segment (start 50.635 155.715) (end 52.6866 157.7666) (width 0.1906) (layer B.Cu) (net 11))
 (segment (start 52.6866 157.7666) (end 52.6866 159.4642) (width 0.1906) (layer B.Cu) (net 11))
 (segment (start 53.81 161.43) (end 53.81 160.552116) (width 0.1905) (layer B.Cu) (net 11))
 (segment (start 53.81 160.5876) (end 53.4692 160.2468) (width 0.1905) (layer B.Cu) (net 11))
 (segment (start 53.81 161.43) (end 53.81 160.5876) (width 0.1905) (layer B.Cu) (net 11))
 (segment (start 52.6866 159.4642) (end 53.4692 160.2468) (width 0.1906) (layer B.Cu) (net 11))
 (segment (start 49.365 156.985) (end 47.6949 158.6551) (width 0.1906) (layer B.Cu) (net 10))
 (segment (start 47.6949 158.6551) (end 47.6949 160.8465) (width 0.1906) (layer B.Cu) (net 10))
 (segment (start 47.6949 160.8465) (end 47.5105 161.0309) (width 0.1906) (layer B.Cu) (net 10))
 (segment (start 47.5105 162.6495) (end 47.5105 161.3535) (width 0.1905) (layer B.Cu) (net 10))
 (segment (start 46.19 163.97) (end 47.5105 162.6495) (width 0.1905) (layer B.Cu) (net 10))
 (segment (start 47.5105 161.0309) (end 47.5105 161.3535) (width 0.1906) (layer B.Cu) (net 10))
 (segment (start 52.4895 160.8164) (end 52.2749 160.6018) (width 0.1906) (layer B.Cu) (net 9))
 (segment (start 52.2749 160.6018) (end 52.2749 158.6249) (width 0.1906) (layer B.Cu) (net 9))
 (segment (start 52.2749 158.6249) (end 50.635 156.985) (width 0.1906) (layer B.Cu) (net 9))
 (segment (start 52.4895 162.6495) (end 52.4895 161.0995) (width 0.1905) (layer B.Cu) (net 9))
 (segment (start 53.81 163.97) (end 52.4895 162.6495) (width 0.1905) (layer B.Cu) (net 9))
 (segment (start 52.4895 161.0995) (end 52.4895 160.8164) (width 0.1906) (layer B.Cu) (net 9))
 (segment (start 49.365 158.255) (end 48.1926 159.4274) (width 0.1906) (layer B.Cu) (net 8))
 (segment (start 48.1926 159.4274) (end 48.1926 160.8703) (width 0.1906) (layer B.Cu) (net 8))
 (segment (start 48.1926 160.8703) (end 47.8792 161.1837) (width 0.1906) (layer B.Cu) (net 8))
 (segment (start 47.8792 161.1837) (end 47.8792 163.9782) (width 0.1906) (layer B.Cu) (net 8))
 (segment (start 46.19 165.6674) (end 46.6577 165.1997) (width 0.1905) (layer B.Cu) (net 8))
 (segment (start 46.19 166.51) (end 46.19 165.6674) (width 0.1905) (layer B.Cu) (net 8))
 (segment (start 47.8792 163.9782) (end 46.6577 165.1997) (width 0.1906) (layer B.Cu) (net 8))
 (segment (start 52.1208 163.9782) (end 52.1208 161.1837) (width 0.1906) (layer B.Cu) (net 7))
 (segment (start 52.1208 161.1837) (end 51.8075 160.8704) (width 0.1906) (layer B.Cu) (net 7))
 (segment (start 51.8075 160.8704) (end 51.8075 159.4275) (width 0.1906) (layer B.Cu) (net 7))
 (segment (start 51.8075 159.4275) (end 50.635 158.255) (width 0.1906) (layer B.Cu) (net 7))
 (segment (start 53.81 165.6674) (end 53.4058 165.2632) (width 0.1905) (layer B.Cu) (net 7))
 (segment (start 53.81 166.51) (end 53.81 165.6674) (width 0.1905) (layer B.Cu) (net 7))
 (segment (start 53.4058 165.2632) (end 52.1208 163.9782) (width 0.1906) (layer B.Cu) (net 7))
 (segment (start 49.365 159.525) (end 48.6166 160.2734) (width 0.1906) (layer B.Cu) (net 6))
 (segment (start 48.6166 160.2734) (end 48.6166 160.9678) (width 0.1906) (layer B.Cu) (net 6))
 (segment (start 48.6166 160.9678) (end 48.2479 161.3365) (width 0.1906) (layer B.Cu) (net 6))
 (segment (start 48.2479 161.3365) (end 48.2479 166.1495) (width 0.1906) (layer B.Cu) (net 6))
 (segment (start 46.19 168.2074) (end 46.6577 167.7397) (width 0.1905) (layer B.Cu) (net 6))
 (segment (start 46.19 169.05) (end 46.19 168.2074) (width 0.1905) (layer B.Cu) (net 6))
 (segment (start 48.2479 166.1495) (end 46.6577 167.7397) (width 0.1906) (layer B.Cu) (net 6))
 (segment (start 51.7521 166.0869) (end 51.7521 161.3365) (width 0.1906) (layer B.Cu) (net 5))
 (segment (start 51.7521 161.3365) (end 51.3834 160.9678) (width 0.1906) (layer B.Cu) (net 5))
 (segment (start 51.3834 160.9678) (end 51.3834 160.2734) (width 0.1906) (layer B.Cu) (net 5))
 (segment (start 51.3834 160.2734) (end 50.635 159.525) (width 0.1906) (layer B.Cu) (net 5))
 (segment (start 53.81 168.1448) (end 53.4371 167.7719) (width 0.1905) (layer B.Cu) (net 5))
 (segment (start 53.81 169.05) (end 53.81 168.1448) (width 0.1905) (layer B.Cu) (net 5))
 (segment (start 53.4371 167.7719) (end 51.7521 166.0869) (width 0.1906) (layer B.Cu) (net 5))
 (segment (start 49.365 160.795) (end 48.6166 161.5434) (width 0.1906) (layer B.Cu) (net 4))
 (segment (start 48.6166 161.5434) (end 48.6166 168.3208) (width 0.1906) (layer B.Cu) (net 4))
 (segment (start 46.19 170.7474) (end 46.5307 170.4067) (width 0.1905) (layer B.Cu) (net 4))
 (segment (start 46.19 171.59) (end 46.19 170.7474) (width 0.1905) (layer B.Cu) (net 4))
 (segment (start 48.6166 168.3208) (end 46.5307 170.4067) (width 0.1906) (layer B.Cu) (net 4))
 (segment (start 51.3834 168.3208) (end 51.3834 161.5434) (width 0.1906) (layer B.Cu) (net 3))
 (segment (start 51.3834 161.5434) (end 50.635 160.795) (width 0.1906) (layer B.Cu) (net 3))
 (segment (start 53.81 170.7474) (end 53.4058 170.3432) (width 0.1905) (layer B.Cu) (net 3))
 (segment (start 53.81 171.59) (end 53.81 170.7474) (width 0.1905) (layer B.Cu) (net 3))
 (segment (start 53.4058 170.3432) (end 51.3834 168.3208) (width 0.1906) (layer B.Cu) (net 3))
 (segment (start 46.19 174.13) (end 47.313051 173.006949) (width 0.1905) (layer B.Cu) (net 2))
 (segment (start 49.365 168.093338) (end 49.365 167.907) (width 0.1905) (layer B.Cu) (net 2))
 (segment (start 47.313051 170.145287) (end 49.365 168.093338) (width 0.1905) (layer B.Cu) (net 2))
 (segment (start 47.313051 173.006949) (end 47.313051 170.145287) (width 0.1905) (layer B.Cu) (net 2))
 (segment (start 49.365 162.065) (end 49.365 167.907) (width 0.1906) (layer B.Cu) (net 2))
 (segment (start 52.686949 170.339949) (end 50.635 168.288) (width 0.1905) (layer B.Cu) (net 1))
 (segment (start 52.686949 173.006949) (end 52.686949 170.339949) (width 0.1905) (layer B.Cu) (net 1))
 (segment (start 53.81 174.13) (end 52.686949 173.006949) (width 0.1905) (layer B.Cu) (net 1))
 (segment (start 50.635 162.065) (end 50.635 168.288) (width 0.1906) (layer B.Cu) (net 1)))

